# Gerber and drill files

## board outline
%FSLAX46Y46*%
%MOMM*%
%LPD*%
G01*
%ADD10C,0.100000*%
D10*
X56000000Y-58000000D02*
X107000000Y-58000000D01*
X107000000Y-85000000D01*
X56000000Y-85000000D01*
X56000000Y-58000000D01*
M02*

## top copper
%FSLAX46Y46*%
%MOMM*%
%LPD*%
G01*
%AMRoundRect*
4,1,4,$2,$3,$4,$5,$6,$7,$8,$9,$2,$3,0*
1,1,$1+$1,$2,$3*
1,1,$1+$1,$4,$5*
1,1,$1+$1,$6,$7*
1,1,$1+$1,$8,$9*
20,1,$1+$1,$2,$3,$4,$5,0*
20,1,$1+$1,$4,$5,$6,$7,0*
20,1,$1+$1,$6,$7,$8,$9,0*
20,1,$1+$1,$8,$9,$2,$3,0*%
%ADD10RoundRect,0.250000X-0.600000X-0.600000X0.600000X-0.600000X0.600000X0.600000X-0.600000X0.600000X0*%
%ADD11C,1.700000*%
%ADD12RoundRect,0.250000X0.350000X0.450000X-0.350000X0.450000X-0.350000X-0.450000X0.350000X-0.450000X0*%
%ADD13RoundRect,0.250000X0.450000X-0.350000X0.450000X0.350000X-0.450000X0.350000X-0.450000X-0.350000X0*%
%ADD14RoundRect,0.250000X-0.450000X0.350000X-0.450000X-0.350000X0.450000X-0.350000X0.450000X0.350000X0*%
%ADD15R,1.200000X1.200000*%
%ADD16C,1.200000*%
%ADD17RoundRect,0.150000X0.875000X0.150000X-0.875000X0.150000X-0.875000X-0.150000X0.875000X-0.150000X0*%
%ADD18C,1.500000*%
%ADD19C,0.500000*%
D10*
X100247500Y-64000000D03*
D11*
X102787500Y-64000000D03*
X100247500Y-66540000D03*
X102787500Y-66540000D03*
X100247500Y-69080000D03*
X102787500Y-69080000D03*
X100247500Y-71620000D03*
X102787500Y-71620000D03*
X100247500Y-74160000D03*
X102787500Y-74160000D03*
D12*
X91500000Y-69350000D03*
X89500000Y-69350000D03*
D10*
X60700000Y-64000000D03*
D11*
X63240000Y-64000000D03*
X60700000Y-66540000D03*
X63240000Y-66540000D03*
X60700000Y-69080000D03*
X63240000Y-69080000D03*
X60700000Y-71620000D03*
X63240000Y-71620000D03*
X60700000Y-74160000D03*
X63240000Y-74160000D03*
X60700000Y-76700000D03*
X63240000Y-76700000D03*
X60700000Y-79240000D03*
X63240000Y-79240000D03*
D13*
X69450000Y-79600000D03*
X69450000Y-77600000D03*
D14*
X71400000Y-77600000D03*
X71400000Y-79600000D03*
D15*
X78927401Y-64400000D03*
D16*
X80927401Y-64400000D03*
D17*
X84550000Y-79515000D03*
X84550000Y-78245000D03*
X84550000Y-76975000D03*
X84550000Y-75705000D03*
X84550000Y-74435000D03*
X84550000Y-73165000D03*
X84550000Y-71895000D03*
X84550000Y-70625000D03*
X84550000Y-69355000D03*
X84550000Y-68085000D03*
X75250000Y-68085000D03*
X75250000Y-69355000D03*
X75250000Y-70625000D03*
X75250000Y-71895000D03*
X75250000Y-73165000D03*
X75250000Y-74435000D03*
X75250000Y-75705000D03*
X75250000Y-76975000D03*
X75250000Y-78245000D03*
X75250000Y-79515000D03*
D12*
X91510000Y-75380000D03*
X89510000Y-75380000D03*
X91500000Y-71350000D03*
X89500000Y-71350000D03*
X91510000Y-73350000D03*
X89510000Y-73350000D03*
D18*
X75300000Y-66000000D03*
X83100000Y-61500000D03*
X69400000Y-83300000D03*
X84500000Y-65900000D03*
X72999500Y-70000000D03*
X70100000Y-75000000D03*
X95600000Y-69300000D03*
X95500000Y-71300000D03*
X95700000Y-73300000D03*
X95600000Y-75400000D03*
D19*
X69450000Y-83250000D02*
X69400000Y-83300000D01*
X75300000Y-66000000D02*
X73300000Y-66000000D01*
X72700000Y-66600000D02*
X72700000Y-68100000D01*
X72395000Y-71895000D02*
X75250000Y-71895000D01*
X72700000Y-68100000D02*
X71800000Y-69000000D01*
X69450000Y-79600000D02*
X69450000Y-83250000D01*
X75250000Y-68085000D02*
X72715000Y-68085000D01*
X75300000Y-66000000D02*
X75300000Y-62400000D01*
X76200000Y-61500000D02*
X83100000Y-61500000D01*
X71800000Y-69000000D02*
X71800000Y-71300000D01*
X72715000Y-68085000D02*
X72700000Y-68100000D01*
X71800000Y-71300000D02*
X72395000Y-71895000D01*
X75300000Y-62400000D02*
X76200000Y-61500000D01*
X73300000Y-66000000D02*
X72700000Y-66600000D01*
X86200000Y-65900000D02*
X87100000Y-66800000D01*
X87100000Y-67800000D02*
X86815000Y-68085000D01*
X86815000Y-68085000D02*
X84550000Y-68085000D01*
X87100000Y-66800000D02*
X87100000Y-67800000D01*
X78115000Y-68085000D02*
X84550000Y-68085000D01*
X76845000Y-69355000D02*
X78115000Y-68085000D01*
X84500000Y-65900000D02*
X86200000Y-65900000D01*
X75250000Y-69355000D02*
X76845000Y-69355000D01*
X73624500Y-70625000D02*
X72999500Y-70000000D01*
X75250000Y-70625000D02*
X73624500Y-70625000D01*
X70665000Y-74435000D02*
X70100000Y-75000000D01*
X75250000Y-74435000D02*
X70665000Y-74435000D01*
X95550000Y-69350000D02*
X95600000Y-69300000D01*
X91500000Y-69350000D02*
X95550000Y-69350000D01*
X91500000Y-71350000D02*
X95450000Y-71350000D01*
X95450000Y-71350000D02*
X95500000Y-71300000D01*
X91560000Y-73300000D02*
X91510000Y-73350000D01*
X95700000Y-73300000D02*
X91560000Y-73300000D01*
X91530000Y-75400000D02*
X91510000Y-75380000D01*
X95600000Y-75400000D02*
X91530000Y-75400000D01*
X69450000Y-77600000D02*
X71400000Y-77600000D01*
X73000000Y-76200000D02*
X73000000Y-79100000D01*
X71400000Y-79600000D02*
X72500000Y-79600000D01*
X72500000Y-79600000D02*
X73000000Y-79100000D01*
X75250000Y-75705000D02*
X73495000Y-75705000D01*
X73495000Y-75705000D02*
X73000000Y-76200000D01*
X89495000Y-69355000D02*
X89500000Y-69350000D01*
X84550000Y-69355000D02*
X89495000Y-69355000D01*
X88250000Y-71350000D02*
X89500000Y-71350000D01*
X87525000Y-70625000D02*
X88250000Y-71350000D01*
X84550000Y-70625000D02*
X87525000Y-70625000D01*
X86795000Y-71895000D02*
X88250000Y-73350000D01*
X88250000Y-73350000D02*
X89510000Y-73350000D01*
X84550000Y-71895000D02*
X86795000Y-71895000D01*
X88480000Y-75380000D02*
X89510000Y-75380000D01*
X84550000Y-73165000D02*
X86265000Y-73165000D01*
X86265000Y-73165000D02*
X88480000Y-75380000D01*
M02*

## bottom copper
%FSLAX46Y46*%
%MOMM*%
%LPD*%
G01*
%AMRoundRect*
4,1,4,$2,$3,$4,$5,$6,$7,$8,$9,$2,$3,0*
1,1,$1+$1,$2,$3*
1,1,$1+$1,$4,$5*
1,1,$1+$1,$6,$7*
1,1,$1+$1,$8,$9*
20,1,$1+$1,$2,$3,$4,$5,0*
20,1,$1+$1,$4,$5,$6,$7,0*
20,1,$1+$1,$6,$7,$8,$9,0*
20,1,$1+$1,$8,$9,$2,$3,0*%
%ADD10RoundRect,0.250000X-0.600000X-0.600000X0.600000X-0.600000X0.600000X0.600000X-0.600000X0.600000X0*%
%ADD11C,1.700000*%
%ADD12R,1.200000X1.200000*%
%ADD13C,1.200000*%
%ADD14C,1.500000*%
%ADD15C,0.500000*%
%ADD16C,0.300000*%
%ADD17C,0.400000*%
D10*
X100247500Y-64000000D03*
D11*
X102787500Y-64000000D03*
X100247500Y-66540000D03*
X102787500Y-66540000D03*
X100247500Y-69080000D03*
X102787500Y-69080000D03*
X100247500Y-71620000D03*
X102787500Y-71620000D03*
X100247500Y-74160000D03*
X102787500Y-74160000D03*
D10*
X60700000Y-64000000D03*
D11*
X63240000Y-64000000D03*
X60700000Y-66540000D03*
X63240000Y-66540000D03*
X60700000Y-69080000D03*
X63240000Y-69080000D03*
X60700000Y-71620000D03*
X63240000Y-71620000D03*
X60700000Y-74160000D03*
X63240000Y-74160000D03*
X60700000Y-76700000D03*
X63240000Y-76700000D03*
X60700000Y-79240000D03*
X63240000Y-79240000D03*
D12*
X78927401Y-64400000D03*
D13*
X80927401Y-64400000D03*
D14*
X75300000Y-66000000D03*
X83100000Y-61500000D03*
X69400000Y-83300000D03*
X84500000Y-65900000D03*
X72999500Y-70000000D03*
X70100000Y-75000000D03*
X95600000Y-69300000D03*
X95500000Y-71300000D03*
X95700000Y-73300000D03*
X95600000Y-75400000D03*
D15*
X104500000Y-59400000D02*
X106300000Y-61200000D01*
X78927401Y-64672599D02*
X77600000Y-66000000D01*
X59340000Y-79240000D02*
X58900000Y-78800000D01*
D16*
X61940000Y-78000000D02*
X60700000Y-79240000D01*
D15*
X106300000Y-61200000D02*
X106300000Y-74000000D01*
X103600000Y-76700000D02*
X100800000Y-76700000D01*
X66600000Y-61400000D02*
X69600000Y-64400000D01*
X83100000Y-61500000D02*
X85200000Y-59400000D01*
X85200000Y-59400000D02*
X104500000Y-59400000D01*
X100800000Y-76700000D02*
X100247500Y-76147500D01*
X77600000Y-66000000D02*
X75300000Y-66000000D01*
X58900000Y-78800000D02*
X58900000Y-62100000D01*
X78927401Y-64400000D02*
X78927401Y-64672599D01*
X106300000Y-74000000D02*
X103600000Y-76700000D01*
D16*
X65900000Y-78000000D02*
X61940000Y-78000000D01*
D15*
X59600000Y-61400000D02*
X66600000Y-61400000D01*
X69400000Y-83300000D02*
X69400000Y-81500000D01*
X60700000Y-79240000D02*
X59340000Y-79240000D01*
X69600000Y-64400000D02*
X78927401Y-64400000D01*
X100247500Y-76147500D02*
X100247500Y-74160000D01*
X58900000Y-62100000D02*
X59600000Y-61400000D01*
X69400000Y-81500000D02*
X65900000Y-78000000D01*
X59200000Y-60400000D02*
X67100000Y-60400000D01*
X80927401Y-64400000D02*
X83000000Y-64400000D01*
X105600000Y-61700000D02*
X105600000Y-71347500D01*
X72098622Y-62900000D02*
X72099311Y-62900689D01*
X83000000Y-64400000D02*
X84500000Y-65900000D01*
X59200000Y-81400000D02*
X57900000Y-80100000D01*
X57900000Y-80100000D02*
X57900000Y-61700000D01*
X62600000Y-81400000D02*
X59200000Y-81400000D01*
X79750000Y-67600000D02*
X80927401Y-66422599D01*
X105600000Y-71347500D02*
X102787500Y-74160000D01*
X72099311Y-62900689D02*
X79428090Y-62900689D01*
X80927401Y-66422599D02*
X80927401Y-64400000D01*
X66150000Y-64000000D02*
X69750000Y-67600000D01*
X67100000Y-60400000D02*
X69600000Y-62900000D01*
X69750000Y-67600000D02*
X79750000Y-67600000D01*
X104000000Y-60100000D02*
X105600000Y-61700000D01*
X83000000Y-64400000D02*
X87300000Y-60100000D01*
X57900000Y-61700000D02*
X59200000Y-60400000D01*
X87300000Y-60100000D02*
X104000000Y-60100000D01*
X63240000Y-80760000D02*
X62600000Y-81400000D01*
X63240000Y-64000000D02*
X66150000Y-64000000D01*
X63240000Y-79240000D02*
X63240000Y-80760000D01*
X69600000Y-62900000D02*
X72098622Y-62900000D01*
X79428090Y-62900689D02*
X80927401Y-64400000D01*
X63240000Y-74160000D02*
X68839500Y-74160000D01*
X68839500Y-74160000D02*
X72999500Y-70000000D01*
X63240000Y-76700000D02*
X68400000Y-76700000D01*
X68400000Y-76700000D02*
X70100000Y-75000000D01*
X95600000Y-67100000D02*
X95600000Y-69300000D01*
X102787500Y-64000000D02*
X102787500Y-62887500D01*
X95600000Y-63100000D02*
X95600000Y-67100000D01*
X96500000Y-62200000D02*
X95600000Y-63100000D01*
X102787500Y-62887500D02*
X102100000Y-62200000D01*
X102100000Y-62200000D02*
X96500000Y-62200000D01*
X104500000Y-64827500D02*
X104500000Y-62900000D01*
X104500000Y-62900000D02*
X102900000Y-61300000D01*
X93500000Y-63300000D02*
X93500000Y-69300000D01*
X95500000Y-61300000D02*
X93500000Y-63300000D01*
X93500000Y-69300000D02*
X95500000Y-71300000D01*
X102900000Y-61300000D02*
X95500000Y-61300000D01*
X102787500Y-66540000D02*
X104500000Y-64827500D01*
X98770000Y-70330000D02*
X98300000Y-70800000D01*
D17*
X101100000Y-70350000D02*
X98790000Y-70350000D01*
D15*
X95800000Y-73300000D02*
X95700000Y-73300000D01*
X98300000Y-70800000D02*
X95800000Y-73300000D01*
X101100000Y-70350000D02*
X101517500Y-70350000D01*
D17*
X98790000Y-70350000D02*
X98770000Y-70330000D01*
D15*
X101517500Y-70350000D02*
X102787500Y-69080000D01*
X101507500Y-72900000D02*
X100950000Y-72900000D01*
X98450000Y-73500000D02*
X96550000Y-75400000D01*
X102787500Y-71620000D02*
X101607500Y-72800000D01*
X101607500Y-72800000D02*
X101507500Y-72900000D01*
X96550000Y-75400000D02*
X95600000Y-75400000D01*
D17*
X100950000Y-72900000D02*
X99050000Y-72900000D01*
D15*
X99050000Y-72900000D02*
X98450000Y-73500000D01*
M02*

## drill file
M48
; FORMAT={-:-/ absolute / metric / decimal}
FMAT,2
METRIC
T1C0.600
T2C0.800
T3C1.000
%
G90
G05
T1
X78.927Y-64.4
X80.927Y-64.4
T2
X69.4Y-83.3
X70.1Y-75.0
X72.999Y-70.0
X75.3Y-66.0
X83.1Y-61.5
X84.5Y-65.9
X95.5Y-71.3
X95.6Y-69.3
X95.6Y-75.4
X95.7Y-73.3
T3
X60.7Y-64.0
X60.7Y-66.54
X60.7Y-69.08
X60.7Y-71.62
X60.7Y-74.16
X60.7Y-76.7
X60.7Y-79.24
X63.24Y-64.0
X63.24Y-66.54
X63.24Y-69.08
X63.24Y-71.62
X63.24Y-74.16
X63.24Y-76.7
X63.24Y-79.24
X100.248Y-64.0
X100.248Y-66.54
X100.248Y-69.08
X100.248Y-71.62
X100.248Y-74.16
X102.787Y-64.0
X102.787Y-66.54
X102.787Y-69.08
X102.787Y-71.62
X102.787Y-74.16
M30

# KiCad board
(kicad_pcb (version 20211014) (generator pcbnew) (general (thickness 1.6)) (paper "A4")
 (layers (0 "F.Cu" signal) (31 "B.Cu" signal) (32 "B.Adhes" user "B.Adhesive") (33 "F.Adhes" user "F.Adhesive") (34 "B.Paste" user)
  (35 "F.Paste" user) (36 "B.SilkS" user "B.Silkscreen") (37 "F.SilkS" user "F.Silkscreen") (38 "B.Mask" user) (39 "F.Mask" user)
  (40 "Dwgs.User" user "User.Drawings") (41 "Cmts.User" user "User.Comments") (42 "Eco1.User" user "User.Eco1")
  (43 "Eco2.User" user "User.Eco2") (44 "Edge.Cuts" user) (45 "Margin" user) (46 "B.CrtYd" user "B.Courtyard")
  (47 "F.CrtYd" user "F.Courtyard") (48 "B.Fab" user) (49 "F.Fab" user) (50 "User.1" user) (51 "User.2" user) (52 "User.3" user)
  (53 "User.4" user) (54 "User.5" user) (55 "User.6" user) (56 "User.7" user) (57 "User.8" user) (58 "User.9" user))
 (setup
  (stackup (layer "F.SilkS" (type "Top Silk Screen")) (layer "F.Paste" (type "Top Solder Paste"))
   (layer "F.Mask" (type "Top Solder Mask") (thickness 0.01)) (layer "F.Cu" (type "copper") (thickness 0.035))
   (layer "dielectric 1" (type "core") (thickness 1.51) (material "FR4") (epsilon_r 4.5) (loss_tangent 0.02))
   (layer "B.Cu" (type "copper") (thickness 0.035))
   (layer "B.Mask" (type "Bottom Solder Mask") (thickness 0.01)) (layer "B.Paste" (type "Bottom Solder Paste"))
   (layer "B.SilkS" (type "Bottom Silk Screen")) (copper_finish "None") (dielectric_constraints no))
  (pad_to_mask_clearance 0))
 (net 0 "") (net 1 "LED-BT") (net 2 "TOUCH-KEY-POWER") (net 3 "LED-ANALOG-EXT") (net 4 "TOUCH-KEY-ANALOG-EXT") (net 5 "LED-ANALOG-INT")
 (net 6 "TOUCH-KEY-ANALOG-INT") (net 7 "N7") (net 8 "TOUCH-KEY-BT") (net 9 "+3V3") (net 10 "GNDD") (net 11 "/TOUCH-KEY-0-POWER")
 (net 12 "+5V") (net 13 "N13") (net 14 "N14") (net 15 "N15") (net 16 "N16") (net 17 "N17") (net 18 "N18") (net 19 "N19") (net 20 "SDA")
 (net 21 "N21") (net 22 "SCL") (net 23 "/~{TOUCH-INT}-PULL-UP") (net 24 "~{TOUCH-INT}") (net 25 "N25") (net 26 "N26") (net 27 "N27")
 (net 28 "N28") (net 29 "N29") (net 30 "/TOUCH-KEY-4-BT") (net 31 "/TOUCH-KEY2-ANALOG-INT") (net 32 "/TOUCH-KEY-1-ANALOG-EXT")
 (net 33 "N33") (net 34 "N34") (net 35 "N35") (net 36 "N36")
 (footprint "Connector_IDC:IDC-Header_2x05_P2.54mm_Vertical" (layer "F.Cu") (at 100.2475 64)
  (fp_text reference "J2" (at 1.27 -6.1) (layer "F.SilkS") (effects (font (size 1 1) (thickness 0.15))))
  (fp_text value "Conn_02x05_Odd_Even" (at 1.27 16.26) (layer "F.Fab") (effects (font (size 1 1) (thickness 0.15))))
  (pad "1" thru_hole roundrect (at 0 0) (size 1.7 1.7) (drill 1) (layers *.Cu *.Mask) (roundrect_rratio 0.1470588235) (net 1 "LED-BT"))
  (pad "2" thru_hole circle (at 2.54 0) (size 1.7 1.7) (drill 1) (layers *.Cu *.Mask) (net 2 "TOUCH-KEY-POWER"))
  (pad "3" thru_hole circle (at 0 2.54) (size 1.7 1.7) (drill 1) (layers *.Cu *.Mask) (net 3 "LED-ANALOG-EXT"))
  (pad "4" thru_hole circle (at 2.54 2.54) (size 1.7 1.7) (drill 1) (layers *.Cu *.Mask) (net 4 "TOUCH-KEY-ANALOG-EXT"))
  (pad "5" thru_hole circle (at 0 5.08) (size 1.7 1.7) (drill 1) (layers *.Cu *.Mask) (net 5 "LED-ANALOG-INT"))
  (pad "6" thru_hole circle (at 2.54 5.08) (size 1.7 1.7) (drill 1) (layers *.Cu *.Mask) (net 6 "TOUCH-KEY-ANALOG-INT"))
  (pad "7" thru_hole circle (at 0 7.62) (size 1.7 1.7) (drill 1) (layers *.Cu *.Mask) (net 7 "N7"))
  (pad "8" thru_hole circle (at 2.54 7.62) (size 1.7 1.7) (drill 1) (layers *.Cu *.Mask) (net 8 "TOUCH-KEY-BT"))
  (pad "9" thru_hole circle (at 0 10.16) (size 1.7 1.7) (drill 1) (layers *.Cu *.Mask) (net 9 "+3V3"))
  (pad "10" thru_hole circle (at 2.54 10.16) (size 1.7 1.7) (drill 1) (layers *.Cu *.Mask) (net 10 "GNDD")))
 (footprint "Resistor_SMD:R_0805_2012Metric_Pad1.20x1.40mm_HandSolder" (layer "F.Cu") (at 90.5 69.35 180)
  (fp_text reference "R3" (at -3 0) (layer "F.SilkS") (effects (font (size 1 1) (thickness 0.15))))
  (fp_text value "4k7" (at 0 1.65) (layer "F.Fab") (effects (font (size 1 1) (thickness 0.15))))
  (pad "1" smd roundrect (at -1 0 180) (size 1.2 1.4) (layers "F.Cu" "F.Paste" "F.Mask") (roundrect_rratio 0.2083333333)
   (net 2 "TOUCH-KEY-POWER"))
  (pad "2" smd roundrect (at 1 0 180) (size 1.2 1.4) (layers "F.Cu" "F.Paste" "F.Mask") (roundrect_rratio 0.2083333333)
   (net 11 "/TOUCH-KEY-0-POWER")))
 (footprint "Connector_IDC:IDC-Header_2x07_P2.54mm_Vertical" (layer "F.Cu") (at 60.7 64)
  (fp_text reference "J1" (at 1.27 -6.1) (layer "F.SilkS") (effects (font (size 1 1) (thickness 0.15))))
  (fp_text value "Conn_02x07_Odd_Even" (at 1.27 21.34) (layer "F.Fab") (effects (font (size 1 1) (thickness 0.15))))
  (pad "1" thru_hole roundrect (at 0 0) (size 1.7 1.7) (drill 1) (layers *.Cu *.Mask) (roundrect_rratio 0.1470588235) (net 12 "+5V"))
  (pad "2" thru_hole circle (at 2.54 0) (size 1.7 1.7) (drill 1) (layers *.Cu *.Mask) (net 10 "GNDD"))
  (pad "3" thru_hole circle (at 0 2.54) (size 1.7 1.7) (drill 1) (layers *.Cu *.Mask) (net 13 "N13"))
  (pad "4" thru_hole circle (at 2.54 2.54) (size 1.7 1.7) (drill 1) (layers *.Cu *.Mask) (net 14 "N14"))
  (pad "5" thru_hole circle (at 0 5.08) (size 1.7 1.7) (drill 1) (layers *.Cu *.Mask) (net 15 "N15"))
  (pad "6" thru_hole circle (at 2.54 5.08) (size 1.7 1.7) (drill 1) (layers *.Cu *.Mask) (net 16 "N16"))
  (pad "7" thru_hole circle (at 0 7.62) (size 1.7 1.7) (drill 1) (layers *.Cu *.Mask) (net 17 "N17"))
  (pad "8" thru_hole circle (at 2.54 7.62) (size 1.7 1.7) (drill 1) (layers *.Cu *.Mask) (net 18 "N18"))
  (pad "9" thru_hole circle (at 0 10.16) (size 1.7 1.7) (drill 1) (layers *.Cu *.Mask) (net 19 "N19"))
  (pad "10" thru_hole circle (at 2.54 10.16) (size 1.7 1.7) (drill 1) (layers *.Cu *.Mask) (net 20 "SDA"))
  (pad "11" thru_hole circle (at 0 12.7) (size 1.7 1.7) (drill 1) (layers *.Cu *.Mask) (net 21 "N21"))
  (pad "12" thru_hole circle (at 2.54 12.7) (size 1.7 1.7) (drill 1) (layers *.Cu *.Mask) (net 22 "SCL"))
  (pad "13" thru_hole circle (at 0 15.24) (size 1.7 1.7) (drill 1) (layers *.Cu *.Mask) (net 9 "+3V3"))
  (pad "14" thru_hole circle (at 2.54 15.24) (size 1.7 1.7) (drill 1) (layers *.Cu *.Mask) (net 10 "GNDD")))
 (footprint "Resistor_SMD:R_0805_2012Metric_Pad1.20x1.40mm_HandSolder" (layer "F.Cu") (at 69.45 78.6 90)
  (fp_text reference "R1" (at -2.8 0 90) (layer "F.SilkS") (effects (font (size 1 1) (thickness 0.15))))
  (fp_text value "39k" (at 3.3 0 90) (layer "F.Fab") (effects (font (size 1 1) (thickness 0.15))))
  (pad "1" smd roundrect (at -1 0 90) (size 1.2 1.4) (layers "F.Cu" "F.Paste" "F.Mask") (roundrect_rratio 0.2083333333) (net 9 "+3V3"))
  (pad "2" smd roundrect (at 1 0 90) (size 1.2 1.4) (layers "F.Cu" "F.Paste" "F.Mask") (roundrect_rratio 0.2083333333)
   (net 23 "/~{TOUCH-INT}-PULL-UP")))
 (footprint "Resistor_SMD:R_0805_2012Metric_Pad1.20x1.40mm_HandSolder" (layer "F.Cu") (at 71.4 78.6 -90)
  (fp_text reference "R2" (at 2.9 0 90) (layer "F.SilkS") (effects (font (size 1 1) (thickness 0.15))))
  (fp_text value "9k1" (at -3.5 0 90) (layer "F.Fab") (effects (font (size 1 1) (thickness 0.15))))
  (pad "1" smd roundrect (at -1 0 270) (size 1.2 1.4) (layers "F.Cu" "F.Paste" "F.Mask") (roundrect_rratio 0.2083333333)
   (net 23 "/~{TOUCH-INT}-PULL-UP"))
  (pad "2" smd roundrect (at 1 0 270) (size 1.2 1.4) (layers "F.Cu" "F.Paste" "F.Mask") (roundrect_rratio 0.2083333333)
   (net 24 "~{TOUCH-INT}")))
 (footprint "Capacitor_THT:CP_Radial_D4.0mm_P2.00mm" (layer "F.Cu") (at 78.927401 64.4)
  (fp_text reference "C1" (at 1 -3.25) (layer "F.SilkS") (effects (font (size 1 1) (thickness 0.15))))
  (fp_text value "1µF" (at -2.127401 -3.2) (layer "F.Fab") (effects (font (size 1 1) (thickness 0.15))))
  (pad "1" thru_hole rect (at 0 0) (size 1.2 1.2) (drill 0.6) (layers *.Cu *.Mask) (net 9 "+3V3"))
  (pad "2" thru_hole circle (at 2 0) (size 1.2 1.2) (drill 0.6) (layers *.Cu *.Mask) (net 10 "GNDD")))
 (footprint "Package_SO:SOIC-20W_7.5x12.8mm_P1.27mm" (layer "F.Cu") (at 79.9 73.8 180)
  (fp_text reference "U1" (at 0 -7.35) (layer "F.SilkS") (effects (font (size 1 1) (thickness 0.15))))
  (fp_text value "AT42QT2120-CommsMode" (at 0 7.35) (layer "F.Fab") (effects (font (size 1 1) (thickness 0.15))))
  (pad "1" smd roundrect (at -4.65 -5.715 180) (size 2.05 0.6) (layers "F.Cu" "F.Paste" "F.Mask") (roundrect_rratio 0.25) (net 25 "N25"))
  (pad "2" smd roundrect (at -4.65 -4.445 180) (size 2.05 0.6) (layers "F.Cu" "F.Paste" "F.Mask") (roundrect_rratio 0.25) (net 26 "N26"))
  (pad "3" smd roundrect (at -4.65 -3.175 180) (size 2.05 0.6) (layers "F.Cu" "F.Paste" "F.Mask") (roundrect_rratio 0.25) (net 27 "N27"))
  (pad "4" smd roundrect (at -4.65 -1.905 180) (size 2.05 0.6) (layers "F.Cu" "F.Paste" "F.Mask") (roundrect_rratio 0.25) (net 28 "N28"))
  (pad "5" smd roundrect (at -4.65 -0.635 180) (size 2.05 0.6) (layers "F.Cu" "F.Paste" "F.Mask") (roundrect_rratio 0.25) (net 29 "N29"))
  (pad "6" smd roundrect (at -4.65 0.635 180) (size 2.05 0.6) (layers "F.Cu" "F.Paste" "F.Mask") (roundrect_rratio 0.25)
   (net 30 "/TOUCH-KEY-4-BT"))
  (pad "7" smd roundrect (at -4.65 1.905 180) (size 2.05 0.6) (layers "F.Cu" "F.Paste" "F.Mask") (roundrect_rratio 0.25)
   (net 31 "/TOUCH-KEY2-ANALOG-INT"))
  (pad "8" smd roundrect (at -4.65 3.175 180) (size 2.05 0.6) (layers "F.Cu" "F.Paste" "F.Mask") (roundrect_rratio 0.25)
   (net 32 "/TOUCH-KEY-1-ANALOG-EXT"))
  (pad "9" smd roundrect (at -4.65 4.445 180) (size 2.05 0.6) (layers "F.Cu" "F.Paste" "F.Mask") (roundrect_rratio 0.25)
   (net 11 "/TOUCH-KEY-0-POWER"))
  (pad "10" smd roundrect (at -4.65 5.715 180) (size 2.05 0.6) (layers "F.Cu" "F.Paste" "F.Mask") (roundrect_rratio 0.25) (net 10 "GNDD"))
  (pad "11" smd roundrect (at 4.65 5.715 180) (size 2.05 0.6) (layers "F.Cu" "F.Paste" "F.Mask") (roundrect_rratio 0.25) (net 9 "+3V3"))
  (pad "12" smd roundrect (at 4.65 4.445 180) (size 2.05 0.6) (layers "F.Cu" "F.Paste" "F.Mask") (roundrect_rratio 0.25) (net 10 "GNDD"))
  (pad "13" smd roundrect (at 4.65 3.175 180) (size 2.05 0.6) (layers "F.Cu" "F.Paste" "F.Mask") (roundrect_rratio 0.25) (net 20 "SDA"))
  (pad "14" smd roundrect (at 4.65 1.905 180) (size 2.05 0.6) (layers "F.Cu" "F.Paste" "F.Mask") (roundrect_rratio 0.25) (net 9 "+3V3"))
  (pad "15" smd roundrect (at 4.65 0.635 180) (size 2.05 0.6) (layers "F.Cu" "F.Paste" "F.Mask") (roundrect_rratio 0.25) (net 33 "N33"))
  (pad "16" smd roundrect (at 4.65 -0.635 180) (size 2.05 0.6) (layers "F.Cu" "F.Paste" "F.Mask") (roundrect_rratio 0.25) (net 22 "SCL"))
  (pad "17" smd roundrect (at 4.65 -1.905 180) (size 2.05 0.6) (layers "F.Cu" "F.Paste" "F.Mask") (roundrect_rratio 0.25)
   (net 24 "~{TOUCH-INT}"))
  (pad "18" smd roundrect (at 4.65 -3.175 180) (size 2.05 0.6) (layers "F.Cu" "F.Paste" "F.Mask") (roundrect_rratio 0.25) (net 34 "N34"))
  (pad "19" smd roundrect (at 4.65 -4.445 180) (size 2.05 0.6) (layers "F.Cu" "F.Paste" "F.Mask") (roundrect_rratio 0.25) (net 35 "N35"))
  (pad "20" smd roundrect (at 4.65 -5.715 180) (size 2.05 0.6) (layers "F.Cu" "F.Paste" "F.Mask") (roundrect_rratio 0.25) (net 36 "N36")))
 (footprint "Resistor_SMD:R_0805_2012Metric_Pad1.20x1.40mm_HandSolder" (layer "F.Cu") (at 90.51 75.38 180)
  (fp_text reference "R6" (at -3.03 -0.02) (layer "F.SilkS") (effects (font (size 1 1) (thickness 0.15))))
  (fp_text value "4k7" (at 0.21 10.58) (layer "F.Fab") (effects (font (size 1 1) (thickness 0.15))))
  (pad "1" smd roundrect (at -1 0 180) (size 1.2 1.4) (layers "F.Cu" "F.Paste" "F.Mask") (roundrect_rratio 0.2083333333)
   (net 8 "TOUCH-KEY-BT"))
  (pad "2" smd roundrect (at 1 0 180) (size 1.2 1.4) (layers "F.Cu" "F.Paste" "F.Mask") (roundrect_rratio 0.2083333333)
   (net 30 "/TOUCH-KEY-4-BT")))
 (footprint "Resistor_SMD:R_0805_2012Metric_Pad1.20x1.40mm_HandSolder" (layer "F.Cu") (at 90.5 71.35 180)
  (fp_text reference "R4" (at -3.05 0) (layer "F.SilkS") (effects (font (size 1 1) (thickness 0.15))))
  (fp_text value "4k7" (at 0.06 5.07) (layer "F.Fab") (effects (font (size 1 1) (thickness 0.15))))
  (pad "1" smd roundrect (at -1 0 180) (size 1.2 1.4) (layers "F.Cu" "F.Paste" "F.Mask") (roundrect_rratio 0.2083333333)
   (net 4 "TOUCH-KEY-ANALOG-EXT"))
  (pad "2" smd roundrect (at 1 0 180) (size 1.2 1.4) (layers "F.Cu" "F.Paste" "F.Mask") (roundrect_rratio 0.2083333333)
   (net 32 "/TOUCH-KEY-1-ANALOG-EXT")))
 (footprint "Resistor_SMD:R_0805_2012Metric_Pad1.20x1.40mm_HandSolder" (layer "F.Cu") (at 90.51 73.35 180)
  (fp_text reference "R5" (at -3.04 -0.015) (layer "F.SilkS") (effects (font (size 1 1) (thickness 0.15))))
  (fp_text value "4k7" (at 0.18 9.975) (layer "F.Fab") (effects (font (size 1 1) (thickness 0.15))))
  (pad "1" smd roundrect (at -1 0 180) (size 1.2 1.4) (layers "F.Cu" "F.Paste" "F.Mask") (roundrect_rratio 0.2083333333)
   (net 6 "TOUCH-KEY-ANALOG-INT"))
  (pad "2" smd roundrect (at 1 0 180) (size 1.2 1.4) (layers "F.Cu" "F.Paste" "F.Mask") (roundrect_rratio 0.2083333333)
   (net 31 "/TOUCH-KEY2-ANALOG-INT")))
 (gr_rect (start 56 58) (end 107 85) (layer "Edge.Cuts") (width 0.1) (fill none))
 (segment (start 69.45 83.25) (end 69.4 83.3) (width 0.5) (layer "F.Cu") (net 9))
 (segment (start 75.3 66) (end 73.3 66) (width 0.5) (layer "F.Cu") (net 9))
 (segment (start 72.7 66.6) (end 72.7 68.1) (width 0.5) (layer "F.Cu") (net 9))
 (segment (start 72.395 71.895) (end 75.25 71.895) (width 0.5) (layer "F.Cu") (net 9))
 (segment (start 72.7 68.1) (end 71.8 69) (width 0.5) (layer "F.Cu") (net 9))
 (segment (start 69.45 79.6) (end 69.45 83.25) (width 0.5) (layer "F.Cu") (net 9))
 (segment (start 75.25 68.085) (end 72.715 68.085) (width 0.5) (layer "F.Cu") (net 9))
 (segment (start 75.3 66) (end 75.3 62.4) (width 0.5) (layer "F.Cu") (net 9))
 (segment (start 76.2 61.5) (end 83.1 61.5) (width 0.5) (layer "F.Cu") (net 9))
 (segment (start 71.8 69) (end 71.8 71.3) (width 0.5) (layer "F.Cu") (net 9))
 (segment (start 72.715 68.085) (end 72.7 68.1) (width 0.5) (layer "F.Cu") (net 9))
 (segment (start 71.8 71.3) (end 72.395 71.895) (width 0.5) (layer "F.Cu") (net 9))
 (segment (start 75.3 62.4) (end 76.2 61.5) (width 0.5) (layer "F.Cu") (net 9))
 (segment (start 73.3 66) (end 72.7 66.6) (width 0.5) (layer "F.Cu") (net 9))
 (via (at 75.3 66) (size 1.5) (drill 0.8) (layers "F.Cu" "B.Cu") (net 9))
 (via (at 83.1 61.5) (size 1.5) (drill 0.8) (layers "F.Cu" "B.Cu") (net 9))
 (via (at 69.4 83.3) (size 1.5) (drill 0.8) (layers "F.Cu" "B.Cu") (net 9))
 (segment (start 104.5 59.4) (end 106.3 61.2) (width 0.5) (layer "B.Cu") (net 9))
 (segment (start 78.927401 64.672599) (end 77.6 66) (width 0.5) (layer "B.Cu") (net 9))
 (segment (start 59.34 79.24) (end 58.9 78.8) (width 0.5) (layer "B.Cu") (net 9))
 (segment (start 61.94 78) (end 60.7 79.24) (width 0.3) (layer "B.Cu") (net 9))
 (segment (start 106.3 61.2) (end 106.3 74) (width 0.5) (layer "B.Cu") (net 9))
 (segment (start 103.6 76.7) (end 100.8 76.7) (width 0.5) (layer "B.Cu") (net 9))
 (segment (start 66.6 61.4) (end 69.6 64.4) (width 0.5) (layer "B.Cu") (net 9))
 (segment (start 83.1 61.5) (end 85.2 59.4) (width 0.5) (layer "B.Cu") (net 9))
 (segment (start 85.2 59.4) (end 104.5 59.4) (width 0.5) (layer "B.Cu") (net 9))
 (segment (start 100.8 76.7) (end 100.2475 76.1475) (width 0.5) (layer "B.Cu") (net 9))
 (segment (start 77.6 66) (end 75.3 66) (width 0.5) (layer "B.Cu") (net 9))
 (segment (start 58.9 78.8) (end 58.9 62.1) (width 0.5) (layer "B.Cu") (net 9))
 (segment (start 78.927401 64.4) (end 78.927401 64.672599) (width 0.5) (layer "B.Cu") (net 9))
 (segment (start 106.3 74) (end 103.6 76.7) (width 0.5) (layer "B.Cu") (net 9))
 (segment (start 65.9 78) (end 61.94 78) (width 0.3) (layer "B.Cu") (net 9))
 (segment (start 59.6 61.4) (end 66.6 61.4) (width 0.5) (layer "B.Cu") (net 9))
 (segment (start 69.4 83.3) (end 69.4 81.5) (width 0.5) (layer "B.Cu") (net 9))
 (segment (start 60.7 79.24) (end 59.34 79.24) (width 0.5) (layer "B.Cu") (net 9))
 (segment (start 69.6 64.4) (end 78.927401 64.4) (width 0.5) (layer "B.Cu") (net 9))
 (segment (start 100.2475 76.1475) (end 100.2475 74.16) (width 0.5) (layer "B.Cu") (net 9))
 (segment (start 58.9 62.1) (end 59.6 61.4) (width 0.5) (layer "B.Cu") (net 9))
 (segment (start 69.4 81.5) (end 65.9 78) (width 0.5) (layer "B.Cu") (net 9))
 (segment (start 86.2 65.9) (end 87.1 66.8) (width 0.5) (layer "F.Cu") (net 10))
 (segment (start 87.1 67.8) (end 86.815 68.085) (width 0.5) (layer "F.Cu") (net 10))
 (segment (start 86.815 68.085) (end 84.55 68.085) (width 0.5) (layer "F.Cu") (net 10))
 (segment (start 87.1 66.8) (end 87.1 67.8) (width 0.5) (layer "F.Cu") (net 10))
 (segment (start 78.115 68.085) (end 84.55 68.085) (width 0.5) (layer "F.Cu") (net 10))
 (segment (start 76.845 69.355) (end 78.115 68.085) (width 0.5) (layer "F.Cu") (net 10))
 (segment (start 84.5 65.9) (end 86.2 65.9) (width 0.5) (layer "F.Cu") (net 10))
 (segment (start 75.25 69.355) (end 76.845 69.355) (width 0.5) (layer "F.Cu") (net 10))
 (via (at 84.5 65.9) (size 1.5) (drill 0.8) (layers "F.Cu" "B.Cu") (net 10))
 (segment (start 59.2 60.4) (end 67.1 60.4) (width 0.5) (layer "B.Cu") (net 10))
 (segment (start 80.927401 64.4) (end 83 64.4) (width 0.5) (layer "B.Cu") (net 10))
 (segment (start 105.6 61.7) (end 105.6 71.3475) (width 0.5) (layer "B.Cu") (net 10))
 (segment (start 72.098622 62.9) (end 72.099311 62.900689) (width 0.5) (layer "B.Cu") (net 10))
 (segment (start 83 64.4) (end 84.5 65.9) (width 0.5) (layer "B.Cu") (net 10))
 (segment (start 59.2 81.4) (end 57.9 80.1) (width 0.5) (layer "B.Cu") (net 10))
 (segment (start 57.9 80.1) (end 57.9 61.7) (width 0.5) (layer "B.Cu") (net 10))
 (segment (start 62.6 81.4) (end 59.2 81.4) (width 0.5) (layer "B.Cu") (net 10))
 (segment (start 79.75 67.6) (end 80.927401 66.422599) (width 0.5) (layer "B.Cu") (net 10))
 (segment (start 105.6 71.3475) (end 102.7875 74.16) (width 0.5) (layer "B.Cu") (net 10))
 (segment (start 72.099311 62.900689) (end 79.42809 62.900689) (width 0.5) (layer "B.Cu") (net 10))
 (segment (start 80.927401 66.422599) (end 80.927401 64.4) (width 0.5) (layer "B.Cu") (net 10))
 (segment (start 66.15 64) (end 69.75 67.6) (width 0.5) (layer "B.Cu") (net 10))
 (segment (start 67.1 60.4) (end 69.6 62.9) (width 0.5) (layer "B.Cu") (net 10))
 (segment (start 69.75 67.6) (end 79.75 67.6) (width 0.5) (layer "B.Cu") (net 10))
 (segment (start 104 60.1) (end 105.6 61.7) (width 0.5) (layer "B.Cu") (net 10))
 (segment (start 83 64.4) (end 87.3 60.1) (width 0.5) (layer "B.Cu") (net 10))
 (segment (start 57.9 61.7) (end 59.2 60.4) (width 0.5) (layer "B.Cu") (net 10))
 (segment (start 87.3 60.1) (end 104 60.1) (width 0.5) (layer "B.Cu") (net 10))
 (segment (start 63.24 80.76) (end 62.6 81.4) (width 0.5) (layer "B.Cu") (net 10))
 (segment (start 63.24 64) (end 66.15 64) (width 0.5) (layer "B.Cu") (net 10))
 (segment (start 63.24 79.24) (end 63.24 80.76) (width 0.5) (layer "B.Cu") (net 10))
 (segment (start 69.6 62.9) (end 72.098622 62.9) (width 0.5) (layer "B.Cu") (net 10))
 (segment (start 79.42809 62.900689) (end 80.927401 64.4) (width 0.5) (layer "B.Cu") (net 10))
 (segment (start 73.6245 70.625) (end 72.9995 70) (width 0.5) (layer "F.Cu") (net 20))
 (segment (start 75.25 70.625) (end 73.6245 70.625) (width 0.5) (layer "F.Cu") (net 20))
 (via (at 72.9995 70) (size 1.5) (drill 0.8) (layers "F.Cu" "B.Cu") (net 20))
 (segment (start 63.24 74.16) (end 68.8395 74.16) (width 0.5) (layer "B.Cu") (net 20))
 (segment (start 68.8395 74.16) (end 72.9995 70) (width 0.5) (layer "B.Cu") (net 20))
 (segment (start 70.665 74.435) (end 70.1 75) (width 0.5) (layer "F.Cu") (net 22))
 (segment (start 75.25 74.435) (end 70.665 74.435) (width 0.5) (layer "F.Cu") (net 22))
 (via (at 70.1 75) (size 1.5) (drill 0.8) (layers "F.Cu" "B.Cu") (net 22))
 (segment (start 63.24 76.7) (end 68.4 76.7) (width 0.5) (layer "B.Cu") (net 22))
 (segment (start 68.4 76.7) (end 70.1 75) (width 0.5) (layer "B.Cu") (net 22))
 (segment (start 95.55 69.35) (end 95.6 69.3) (width 0.5) (layer "F.Cu") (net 2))
 (segment (start 91.5 69.35) (end 95.55 69.35) (width 0.5) (layer "F.Cu") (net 2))
 (via (at 95.6 69.3) (size 1.5) (drill 0.8) (layers "F.Cu" "B.Cu") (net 2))
 (segment (start 95.6 67.1) (end 95.6 69.3) (width 0.5) (layer "B.Cu") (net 2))
 (segment (start 102.7875 64) (end 102.7875 62.8875) (width 0.5) (layer "B.Cu") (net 2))
 (segment (start 95.6 63.1) (end 95.6 67.1) (width 0.5) (layer "B.Cu") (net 2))
 (segment (start 96.5 62.2) (end 95.6 63.1) (width 0.5) (layer "B.Cu") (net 2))
 (segment (start 102.7875 62.8875) (end 102.1 62.2) (width 0.5) (layer "B.Cu") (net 2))
 (segment (start 102.1 62.2) (end 96.5 62.2) (width 0.5) (layer "B.Cu") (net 2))
 (segment (start 91.5 71.35) (end 95.45 71.35) (width 0.5) (layer "F.Cu") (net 4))
 (segment (start 95.45 71.35) (end 95.5 71.3) (width 0.5) (layer "F.Cu") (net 4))
 (via (at 95.5 71.3) (size 1.5) (drill 0.8) (layers "F.Cu" "B.Cu") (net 4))
 (segment (start 104.5 64.8275) (end 104.5 62.9) (width 0.5) (layer "B.Cu") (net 4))
 (segment (start 104.5 62.9) (end 102.9 61.3) (width 0.5) (layer "B.Cu") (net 4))
 (segment (start 93.5 63.3) (end 93.5 69.3) (width 0.5) (layer "B.Cu") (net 4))
 (segment (start 95.5 61.3) (end 93.5 63.3) (width 0.5) (layer "B.Cu") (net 4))
 (segment (start 93.5 69.3) (end 95.5 71.3) (width 0.5) (layer "B.Cu") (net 4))
 (segment (start 102.9 61.3) (end 95.5 61.3) (width 0.5) (layer "B.Cu") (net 4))
 (segment (start 102.7875 66.54) (end 104.5 64.8275) (width 0.5) (layer "B.Cu") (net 4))
 (segment (start 91.56 73.3) (end 91.51 73.35) (width 0.5) (layer "F.Cu") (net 6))
 (segment (start 95.7 73.3) (end 91.56 73.3) (width 0.5) (layer "F.Cu") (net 6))
 (via (at 95.7 73.3) (size 1.5) (drill 0.8) (layers "F.Cu" "B.Cu") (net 6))
 (segment (start 98.77 70.33) (end 98.3 70.8) (width 0.5) (layer "B.Cu") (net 6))
 (segment (start 101.1 70.35) (end 98.79 70.35) (width 0.4) (layer "B.Cu") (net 6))
 (segment (start 95.8 73.3) (end 95.7 73.3) (width 0.5) (layer "B.Cu") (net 6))
 (segment (start 98.3 70.8) (end 95.8 73.3) (width 0.5) (layer "B.Cu") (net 6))
 (segment (start 101.1 70.35) (end 101.5175 70.35) (width 0.5) (layer "B.Cu") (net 6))
 (segment (start 98.79 70.35) (end 98.77 70.33) (width 0.4) (layer "B.Cu") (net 6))
 (segment (start 101.5175 70.35) (end 102.7875 69.08) (width 0.5) (layer "B.Cu") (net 6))
 (segment (start 91.53 75.4) (end 91.51 75.38) (width 0.5) (layer "F.Cu") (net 8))
 (segment (start 95.6 75.4) (end 91.53 75.4) (width 0.5) (layer "F.Cu") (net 8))
 (via (at 95.6 75.4) (size 1.5) (drill 0.8) (layers "F.Cu" "B.Cu") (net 8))
 (segment (start 101.5075 72.9) (end 100.95 72.9) (width 0.5) (layer "B.Cu") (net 8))
 (segment (start 98.45 73.5) (end 96.55 75.4) (width 0.5) (layer "B.Cu") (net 8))
 (segment (start 102.7875 71.62) (end 101.6075 72.8) (width 0.5) (layer "B.Cu") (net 8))
 (segment (start 101.6075 72.8) (end 101.5075 72.9) (width 0.5) (layer "B.Cu") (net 8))
 (segment (start 96.55 75.4) (end 95.6 75.4) (width 0.5) (layer "B.Cu") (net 8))
 (segment (start 100.95 72.9) (end 99.05 72.9) (width 0.4) (layer "B.Cu") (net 8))
 (segment (start 99.05 72.9) (end 98.45 73.5) (width 0.5) (layer "B.Cu") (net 8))
 (segment (start 69.45 77.6) (end 71.4 77.6) (width 0.5) (layer "F.Cu") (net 23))
 (segment (start 73 76.2) (end 73 79.1) (width 0.5) (layer "F.Cu") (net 24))
 (segment (start 71.4 79.6) (end 72.5 79.6) (width 0.5) (layer "F.Cu") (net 24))
 (segment (start 72.5 79.6) (end 73 79.1) (width 0.5) (layer "F.Cu") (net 24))
 (segment (start 75.25 75.705) (end 73.495 75.705) (width 0.5) (layer "F.Cu") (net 24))
 (segment (start 73.495 75.705) (end 73 76.2) (width 0.5) (layer "F.Cu") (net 24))
 (segment (start 89.495 69.355) (end 89.5 69.35) (width 0.5) (layer "F.Cu") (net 11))
 (segment (start 84.55 69.355) (end 89.495 69.355) (width 0.5) (layer "F.Cu") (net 11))
 (segment (start 88.25 71.35) (end 89.5 71.35) (width 0.5) (layer "F.Cu") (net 32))
 (segment (start 87.525 70.625) (end 88.25 71.35) (width 0.5) (layer "F.Cu") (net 32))
 (segment (start 84.55 70.625) (end 87.525 70.625) (width 0.5) (layer "F.Cu") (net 32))
 (segment (start 86.795 71.895) (end 88.25 73.35) (width 0.5) (layer "F.Cu") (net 31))
 (segment (start 88.25 73.35) (end 89.51 73.35) (width 0.5) (layer "F.Cu") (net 31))
 (segment (start 84.55 71.895) (end 86.795 71.895) (width 0.5) (layer "F.Cu") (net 31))
 (segment (start 88.48 75.38) (end 89.51 75.38) (width 0.5) (layer "F.Cu") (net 30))
 (segment (start 84.55 73.165) (end 86.265 73.165) (width 0.5) (layer "F.Cu") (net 30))
 (segment (start 86.265 73.165) (end 88.48 75.38) (width 0.5) (layer "F.Cu") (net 30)))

